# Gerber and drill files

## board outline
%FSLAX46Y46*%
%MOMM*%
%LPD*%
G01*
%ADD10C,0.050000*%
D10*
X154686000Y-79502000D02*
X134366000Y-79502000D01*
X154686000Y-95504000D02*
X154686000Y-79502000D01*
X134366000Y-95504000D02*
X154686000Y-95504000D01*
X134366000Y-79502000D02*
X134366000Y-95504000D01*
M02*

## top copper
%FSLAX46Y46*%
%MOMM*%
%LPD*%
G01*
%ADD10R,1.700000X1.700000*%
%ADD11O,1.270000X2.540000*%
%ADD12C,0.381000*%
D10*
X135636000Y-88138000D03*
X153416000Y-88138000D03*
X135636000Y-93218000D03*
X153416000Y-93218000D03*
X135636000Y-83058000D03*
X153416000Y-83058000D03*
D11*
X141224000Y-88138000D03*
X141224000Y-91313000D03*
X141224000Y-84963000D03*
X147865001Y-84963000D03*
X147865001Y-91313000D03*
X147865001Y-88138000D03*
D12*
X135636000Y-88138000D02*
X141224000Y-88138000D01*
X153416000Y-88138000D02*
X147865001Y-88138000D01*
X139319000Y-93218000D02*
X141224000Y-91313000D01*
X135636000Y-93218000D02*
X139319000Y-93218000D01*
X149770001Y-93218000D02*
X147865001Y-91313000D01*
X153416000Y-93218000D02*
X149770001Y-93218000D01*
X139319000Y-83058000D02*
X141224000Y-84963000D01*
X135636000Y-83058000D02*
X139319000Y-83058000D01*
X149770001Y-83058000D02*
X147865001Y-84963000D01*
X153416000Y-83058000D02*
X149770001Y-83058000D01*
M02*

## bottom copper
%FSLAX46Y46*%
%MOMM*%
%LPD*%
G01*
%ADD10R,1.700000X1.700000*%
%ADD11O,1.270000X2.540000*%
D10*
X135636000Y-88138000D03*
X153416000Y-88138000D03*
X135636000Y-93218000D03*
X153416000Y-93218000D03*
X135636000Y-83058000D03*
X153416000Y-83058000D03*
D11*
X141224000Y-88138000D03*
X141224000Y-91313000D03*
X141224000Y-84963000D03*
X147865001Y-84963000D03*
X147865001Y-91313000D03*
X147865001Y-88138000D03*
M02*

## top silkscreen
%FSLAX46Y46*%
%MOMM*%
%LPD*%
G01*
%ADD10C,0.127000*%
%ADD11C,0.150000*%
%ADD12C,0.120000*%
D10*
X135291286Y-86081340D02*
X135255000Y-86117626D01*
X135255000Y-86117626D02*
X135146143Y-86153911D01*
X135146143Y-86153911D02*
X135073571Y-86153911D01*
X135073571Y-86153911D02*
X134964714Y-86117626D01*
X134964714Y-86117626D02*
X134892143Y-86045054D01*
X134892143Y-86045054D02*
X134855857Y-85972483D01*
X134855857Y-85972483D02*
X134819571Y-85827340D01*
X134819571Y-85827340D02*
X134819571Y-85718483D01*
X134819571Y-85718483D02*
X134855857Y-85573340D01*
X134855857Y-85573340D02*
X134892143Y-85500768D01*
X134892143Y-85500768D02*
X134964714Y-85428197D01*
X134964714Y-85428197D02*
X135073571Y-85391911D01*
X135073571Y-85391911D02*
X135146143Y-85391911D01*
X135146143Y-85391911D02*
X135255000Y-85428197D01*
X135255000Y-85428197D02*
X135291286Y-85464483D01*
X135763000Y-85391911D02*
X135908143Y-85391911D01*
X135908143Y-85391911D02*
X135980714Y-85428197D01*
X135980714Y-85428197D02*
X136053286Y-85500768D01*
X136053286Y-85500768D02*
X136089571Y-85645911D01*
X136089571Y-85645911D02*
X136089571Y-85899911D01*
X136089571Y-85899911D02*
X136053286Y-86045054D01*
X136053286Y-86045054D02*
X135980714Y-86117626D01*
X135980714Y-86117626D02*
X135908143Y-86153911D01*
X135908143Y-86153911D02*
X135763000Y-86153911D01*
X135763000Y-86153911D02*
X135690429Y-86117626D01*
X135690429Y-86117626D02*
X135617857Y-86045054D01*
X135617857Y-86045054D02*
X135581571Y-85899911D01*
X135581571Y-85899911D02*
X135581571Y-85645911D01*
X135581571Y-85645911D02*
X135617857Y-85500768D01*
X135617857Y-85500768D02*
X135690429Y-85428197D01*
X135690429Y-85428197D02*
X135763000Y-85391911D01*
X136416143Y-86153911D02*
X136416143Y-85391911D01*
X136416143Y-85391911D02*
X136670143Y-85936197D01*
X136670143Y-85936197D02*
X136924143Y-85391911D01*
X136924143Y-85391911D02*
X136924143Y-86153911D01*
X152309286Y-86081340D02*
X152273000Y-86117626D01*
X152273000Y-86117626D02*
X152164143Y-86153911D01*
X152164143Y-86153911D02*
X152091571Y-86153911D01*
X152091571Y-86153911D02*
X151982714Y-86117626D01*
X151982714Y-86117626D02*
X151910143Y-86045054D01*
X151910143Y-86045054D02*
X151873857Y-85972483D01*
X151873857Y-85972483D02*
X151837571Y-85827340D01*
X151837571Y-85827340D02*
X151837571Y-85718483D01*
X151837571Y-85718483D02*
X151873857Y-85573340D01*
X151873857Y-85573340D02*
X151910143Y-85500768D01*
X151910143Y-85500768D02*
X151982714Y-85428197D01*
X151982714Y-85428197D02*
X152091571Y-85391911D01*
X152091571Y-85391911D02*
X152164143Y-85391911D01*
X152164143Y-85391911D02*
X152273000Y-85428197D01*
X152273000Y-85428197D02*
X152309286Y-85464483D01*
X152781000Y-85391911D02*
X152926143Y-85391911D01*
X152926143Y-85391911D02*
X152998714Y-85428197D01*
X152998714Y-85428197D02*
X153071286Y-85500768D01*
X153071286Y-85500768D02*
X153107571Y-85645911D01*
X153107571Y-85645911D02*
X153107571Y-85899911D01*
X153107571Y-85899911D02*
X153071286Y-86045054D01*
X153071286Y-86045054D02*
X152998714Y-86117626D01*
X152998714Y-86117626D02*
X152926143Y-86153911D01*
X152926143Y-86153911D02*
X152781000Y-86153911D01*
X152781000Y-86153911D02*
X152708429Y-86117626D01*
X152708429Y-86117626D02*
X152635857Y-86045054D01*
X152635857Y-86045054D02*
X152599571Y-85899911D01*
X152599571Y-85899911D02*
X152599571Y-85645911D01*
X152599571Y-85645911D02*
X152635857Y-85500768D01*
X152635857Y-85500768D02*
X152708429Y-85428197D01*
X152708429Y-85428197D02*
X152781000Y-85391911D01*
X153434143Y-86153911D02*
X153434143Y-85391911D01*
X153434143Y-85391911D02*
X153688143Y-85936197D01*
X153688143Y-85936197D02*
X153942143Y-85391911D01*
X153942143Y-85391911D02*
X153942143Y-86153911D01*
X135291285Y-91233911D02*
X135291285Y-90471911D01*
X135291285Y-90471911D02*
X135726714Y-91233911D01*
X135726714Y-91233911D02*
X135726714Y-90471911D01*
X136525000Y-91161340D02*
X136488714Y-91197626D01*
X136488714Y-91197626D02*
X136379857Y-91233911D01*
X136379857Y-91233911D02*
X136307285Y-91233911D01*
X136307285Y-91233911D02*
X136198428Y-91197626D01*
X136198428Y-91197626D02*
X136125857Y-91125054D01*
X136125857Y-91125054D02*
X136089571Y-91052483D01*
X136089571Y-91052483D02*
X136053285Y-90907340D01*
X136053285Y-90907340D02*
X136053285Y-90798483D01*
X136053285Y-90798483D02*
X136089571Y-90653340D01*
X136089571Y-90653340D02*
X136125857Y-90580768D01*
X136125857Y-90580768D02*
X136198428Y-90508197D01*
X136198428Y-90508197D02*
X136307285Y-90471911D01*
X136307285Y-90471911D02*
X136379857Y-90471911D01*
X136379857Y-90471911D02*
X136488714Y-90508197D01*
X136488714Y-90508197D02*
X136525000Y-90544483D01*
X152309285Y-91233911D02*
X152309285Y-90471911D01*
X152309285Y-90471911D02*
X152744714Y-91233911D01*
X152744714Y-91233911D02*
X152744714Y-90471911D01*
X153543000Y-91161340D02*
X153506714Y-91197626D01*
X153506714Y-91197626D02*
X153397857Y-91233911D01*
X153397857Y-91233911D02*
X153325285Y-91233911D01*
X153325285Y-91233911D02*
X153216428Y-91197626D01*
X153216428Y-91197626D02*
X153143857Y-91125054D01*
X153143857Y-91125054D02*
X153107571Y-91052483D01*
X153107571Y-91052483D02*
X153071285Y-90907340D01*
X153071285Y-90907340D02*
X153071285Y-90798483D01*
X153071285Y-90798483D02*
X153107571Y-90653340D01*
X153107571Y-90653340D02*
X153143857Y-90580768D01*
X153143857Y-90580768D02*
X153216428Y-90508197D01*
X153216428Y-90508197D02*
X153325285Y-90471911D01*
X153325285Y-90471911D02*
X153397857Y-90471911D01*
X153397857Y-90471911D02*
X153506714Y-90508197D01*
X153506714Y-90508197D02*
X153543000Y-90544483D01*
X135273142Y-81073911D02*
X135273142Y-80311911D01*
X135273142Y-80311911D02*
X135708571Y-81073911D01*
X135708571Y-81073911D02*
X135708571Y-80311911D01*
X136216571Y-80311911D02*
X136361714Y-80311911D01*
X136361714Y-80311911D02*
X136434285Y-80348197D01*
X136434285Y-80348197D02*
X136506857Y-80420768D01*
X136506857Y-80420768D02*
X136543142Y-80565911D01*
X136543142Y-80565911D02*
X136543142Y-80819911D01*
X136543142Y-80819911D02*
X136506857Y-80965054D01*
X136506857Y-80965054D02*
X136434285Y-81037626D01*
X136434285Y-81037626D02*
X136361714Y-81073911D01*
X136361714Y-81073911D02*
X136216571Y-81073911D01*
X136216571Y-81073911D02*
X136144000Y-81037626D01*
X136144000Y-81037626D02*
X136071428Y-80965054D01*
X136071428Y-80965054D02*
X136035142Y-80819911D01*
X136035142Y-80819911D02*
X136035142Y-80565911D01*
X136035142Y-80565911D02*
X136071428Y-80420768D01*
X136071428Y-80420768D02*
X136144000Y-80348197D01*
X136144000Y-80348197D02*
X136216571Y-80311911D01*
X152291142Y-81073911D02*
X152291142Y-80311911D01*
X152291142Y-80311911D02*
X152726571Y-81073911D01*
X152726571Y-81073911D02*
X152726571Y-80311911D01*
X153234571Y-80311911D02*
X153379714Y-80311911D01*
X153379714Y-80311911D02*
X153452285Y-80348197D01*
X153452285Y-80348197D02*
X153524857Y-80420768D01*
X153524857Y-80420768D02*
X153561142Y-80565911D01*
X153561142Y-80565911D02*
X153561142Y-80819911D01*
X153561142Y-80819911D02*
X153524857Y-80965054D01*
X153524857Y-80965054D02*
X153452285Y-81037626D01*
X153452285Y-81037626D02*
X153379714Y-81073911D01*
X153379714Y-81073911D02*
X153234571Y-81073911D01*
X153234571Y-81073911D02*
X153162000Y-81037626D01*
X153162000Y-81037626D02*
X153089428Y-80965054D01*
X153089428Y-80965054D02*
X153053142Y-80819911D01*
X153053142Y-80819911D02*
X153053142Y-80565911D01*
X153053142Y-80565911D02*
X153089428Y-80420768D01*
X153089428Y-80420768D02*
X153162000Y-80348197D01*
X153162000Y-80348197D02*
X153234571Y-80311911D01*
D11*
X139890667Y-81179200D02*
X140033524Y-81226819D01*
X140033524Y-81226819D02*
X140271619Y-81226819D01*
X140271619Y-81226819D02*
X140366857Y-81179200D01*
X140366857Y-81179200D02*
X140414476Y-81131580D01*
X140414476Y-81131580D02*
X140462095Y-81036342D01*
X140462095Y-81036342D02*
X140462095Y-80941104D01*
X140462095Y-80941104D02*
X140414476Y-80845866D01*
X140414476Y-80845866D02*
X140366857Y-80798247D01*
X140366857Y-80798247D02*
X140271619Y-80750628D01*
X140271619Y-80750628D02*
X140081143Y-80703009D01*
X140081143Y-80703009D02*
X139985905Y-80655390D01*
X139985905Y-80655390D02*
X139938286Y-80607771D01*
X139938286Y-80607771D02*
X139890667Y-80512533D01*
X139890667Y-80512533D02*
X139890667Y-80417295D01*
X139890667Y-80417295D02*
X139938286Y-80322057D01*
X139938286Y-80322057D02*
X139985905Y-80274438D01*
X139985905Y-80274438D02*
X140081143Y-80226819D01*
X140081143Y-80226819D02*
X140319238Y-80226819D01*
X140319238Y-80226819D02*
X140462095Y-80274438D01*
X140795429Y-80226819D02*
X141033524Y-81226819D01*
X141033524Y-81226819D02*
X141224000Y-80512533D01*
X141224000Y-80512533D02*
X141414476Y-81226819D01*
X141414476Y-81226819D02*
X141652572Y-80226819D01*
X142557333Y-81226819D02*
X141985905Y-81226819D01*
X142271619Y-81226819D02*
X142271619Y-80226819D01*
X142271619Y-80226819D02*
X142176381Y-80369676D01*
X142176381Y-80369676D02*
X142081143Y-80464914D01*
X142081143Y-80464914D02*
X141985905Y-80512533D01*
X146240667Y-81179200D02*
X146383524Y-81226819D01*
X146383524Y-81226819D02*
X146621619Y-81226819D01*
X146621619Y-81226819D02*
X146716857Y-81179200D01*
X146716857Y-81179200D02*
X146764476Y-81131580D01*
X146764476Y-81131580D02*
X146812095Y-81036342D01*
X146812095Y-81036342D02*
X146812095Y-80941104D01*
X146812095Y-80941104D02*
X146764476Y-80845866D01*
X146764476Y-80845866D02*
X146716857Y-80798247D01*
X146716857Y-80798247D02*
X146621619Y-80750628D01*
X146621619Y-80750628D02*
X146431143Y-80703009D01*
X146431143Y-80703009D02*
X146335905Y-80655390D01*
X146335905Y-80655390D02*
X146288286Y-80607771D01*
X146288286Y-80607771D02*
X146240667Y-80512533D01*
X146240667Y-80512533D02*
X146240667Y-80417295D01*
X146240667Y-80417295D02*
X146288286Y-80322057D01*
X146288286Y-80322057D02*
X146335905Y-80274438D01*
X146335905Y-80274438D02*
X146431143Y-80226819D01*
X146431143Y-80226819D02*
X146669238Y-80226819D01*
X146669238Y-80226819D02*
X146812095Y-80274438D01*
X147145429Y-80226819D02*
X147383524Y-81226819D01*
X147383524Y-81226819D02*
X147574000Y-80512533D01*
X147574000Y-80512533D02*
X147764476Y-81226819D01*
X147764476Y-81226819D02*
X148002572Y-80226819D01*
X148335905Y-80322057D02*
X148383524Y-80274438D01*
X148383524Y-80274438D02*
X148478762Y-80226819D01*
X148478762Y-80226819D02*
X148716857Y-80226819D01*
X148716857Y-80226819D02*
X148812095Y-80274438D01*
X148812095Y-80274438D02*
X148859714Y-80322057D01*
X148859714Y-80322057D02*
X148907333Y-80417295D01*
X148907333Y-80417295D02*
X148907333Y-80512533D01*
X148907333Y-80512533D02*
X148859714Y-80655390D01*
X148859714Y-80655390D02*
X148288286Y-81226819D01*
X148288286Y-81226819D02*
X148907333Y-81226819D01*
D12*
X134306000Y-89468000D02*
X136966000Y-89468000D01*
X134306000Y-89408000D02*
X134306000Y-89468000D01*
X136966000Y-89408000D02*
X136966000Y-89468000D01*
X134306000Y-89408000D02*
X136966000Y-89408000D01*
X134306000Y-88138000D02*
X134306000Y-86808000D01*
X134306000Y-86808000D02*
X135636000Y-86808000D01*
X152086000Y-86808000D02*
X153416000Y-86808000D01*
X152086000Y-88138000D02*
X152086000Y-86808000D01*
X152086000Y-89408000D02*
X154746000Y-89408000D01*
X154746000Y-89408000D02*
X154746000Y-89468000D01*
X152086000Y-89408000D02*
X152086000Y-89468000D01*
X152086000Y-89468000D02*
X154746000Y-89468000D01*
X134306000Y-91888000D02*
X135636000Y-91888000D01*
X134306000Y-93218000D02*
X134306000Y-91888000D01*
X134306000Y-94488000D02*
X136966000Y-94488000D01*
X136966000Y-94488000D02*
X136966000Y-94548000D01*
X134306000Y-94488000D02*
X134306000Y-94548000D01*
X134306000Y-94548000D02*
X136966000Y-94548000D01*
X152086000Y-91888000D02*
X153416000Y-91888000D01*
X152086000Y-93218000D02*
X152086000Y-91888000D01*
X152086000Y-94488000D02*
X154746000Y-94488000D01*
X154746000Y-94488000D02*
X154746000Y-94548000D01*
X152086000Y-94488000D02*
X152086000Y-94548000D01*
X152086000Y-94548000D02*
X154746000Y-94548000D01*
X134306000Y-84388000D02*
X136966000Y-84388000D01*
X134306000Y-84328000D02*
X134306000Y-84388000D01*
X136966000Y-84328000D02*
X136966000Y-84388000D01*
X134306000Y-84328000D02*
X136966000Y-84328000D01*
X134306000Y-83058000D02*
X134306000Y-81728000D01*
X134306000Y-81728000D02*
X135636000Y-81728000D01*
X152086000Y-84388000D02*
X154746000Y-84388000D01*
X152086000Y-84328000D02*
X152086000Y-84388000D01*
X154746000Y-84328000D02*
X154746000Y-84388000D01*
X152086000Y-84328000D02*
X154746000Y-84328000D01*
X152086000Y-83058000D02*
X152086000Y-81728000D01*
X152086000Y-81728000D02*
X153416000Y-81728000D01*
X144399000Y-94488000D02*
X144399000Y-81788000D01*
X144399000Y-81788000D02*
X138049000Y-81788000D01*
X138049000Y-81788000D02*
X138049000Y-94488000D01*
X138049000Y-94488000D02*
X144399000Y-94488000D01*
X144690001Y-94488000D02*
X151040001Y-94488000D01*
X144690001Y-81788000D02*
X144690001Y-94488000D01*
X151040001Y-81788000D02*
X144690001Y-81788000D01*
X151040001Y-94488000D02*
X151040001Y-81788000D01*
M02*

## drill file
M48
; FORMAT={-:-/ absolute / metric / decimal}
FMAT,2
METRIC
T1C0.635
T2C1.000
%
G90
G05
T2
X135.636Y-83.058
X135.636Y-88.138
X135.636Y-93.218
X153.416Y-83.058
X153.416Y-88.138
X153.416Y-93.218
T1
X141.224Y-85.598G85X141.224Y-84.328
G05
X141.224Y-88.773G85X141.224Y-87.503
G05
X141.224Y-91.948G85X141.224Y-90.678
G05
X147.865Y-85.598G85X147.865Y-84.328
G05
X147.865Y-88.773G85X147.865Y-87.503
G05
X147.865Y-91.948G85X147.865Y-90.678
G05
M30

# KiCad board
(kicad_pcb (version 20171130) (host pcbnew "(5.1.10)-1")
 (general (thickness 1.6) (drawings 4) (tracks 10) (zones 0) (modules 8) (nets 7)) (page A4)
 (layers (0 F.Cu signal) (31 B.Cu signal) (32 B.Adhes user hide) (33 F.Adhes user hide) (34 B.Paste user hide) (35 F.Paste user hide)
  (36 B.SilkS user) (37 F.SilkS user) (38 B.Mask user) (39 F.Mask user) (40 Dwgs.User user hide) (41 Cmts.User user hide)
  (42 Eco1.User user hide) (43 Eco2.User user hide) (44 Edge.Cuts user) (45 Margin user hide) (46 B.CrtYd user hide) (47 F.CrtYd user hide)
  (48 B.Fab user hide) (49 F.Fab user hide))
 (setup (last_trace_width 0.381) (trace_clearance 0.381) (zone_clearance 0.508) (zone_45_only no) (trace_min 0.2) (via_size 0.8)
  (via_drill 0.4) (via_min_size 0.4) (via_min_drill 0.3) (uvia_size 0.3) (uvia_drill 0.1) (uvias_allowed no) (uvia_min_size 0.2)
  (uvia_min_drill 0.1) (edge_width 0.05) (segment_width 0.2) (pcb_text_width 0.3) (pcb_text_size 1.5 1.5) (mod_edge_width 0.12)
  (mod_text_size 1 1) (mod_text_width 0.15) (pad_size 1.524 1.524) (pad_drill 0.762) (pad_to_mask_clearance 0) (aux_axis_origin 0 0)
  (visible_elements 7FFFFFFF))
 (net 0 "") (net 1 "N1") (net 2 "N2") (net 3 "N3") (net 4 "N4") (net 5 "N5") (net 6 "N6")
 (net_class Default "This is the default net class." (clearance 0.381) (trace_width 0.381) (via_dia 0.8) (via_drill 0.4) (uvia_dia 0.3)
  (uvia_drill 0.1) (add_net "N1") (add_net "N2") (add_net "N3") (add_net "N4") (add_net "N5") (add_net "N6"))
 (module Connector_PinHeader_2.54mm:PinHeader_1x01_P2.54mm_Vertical (layer F.Cu) (at 135.636 88.138)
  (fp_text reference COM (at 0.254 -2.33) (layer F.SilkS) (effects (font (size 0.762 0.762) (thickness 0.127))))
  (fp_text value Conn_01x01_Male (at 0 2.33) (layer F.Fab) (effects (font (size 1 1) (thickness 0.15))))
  (fp_line (start -1.33 1.33) (end 1.33 1.33) (layer F.SilkS) (width 0.12))
  (fp_line (start -1.33 1.27) (end -1.33 1.33) (layer F.SilkS) (width 0.12))
  (fp_line (start 1.33 1.27) (end 1.33 1.33) (layer F.SilkS) (width 0.12))
  (fp_line (start -1.33 1.27) (end 1.33 1.27) (layer F.SilkS) (width 0.12))
  (fp_line (start -1.33 0) (end -1.33 -1.33) (layer F.SilkS) (width 0.12))
  (fp_line (start -1.33 -1.33) (end 0 -1.33) (layer F.SilkS) (width 0.12))
  (pad 1 thru_hole rect (at 0 0) (size 1.7 1.7) (drill 1) (layers *.Cu *.Mask) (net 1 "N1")))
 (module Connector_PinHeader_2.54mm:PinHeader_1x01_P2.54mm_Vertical (layer F.Cu) (at 153.416 88.138)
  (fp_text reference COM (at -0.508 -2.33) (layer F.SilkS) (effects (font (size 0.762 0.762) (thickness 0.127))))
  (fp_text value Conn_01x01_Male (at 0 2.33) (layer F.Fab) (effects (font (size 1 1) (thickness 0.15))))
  (fp_line (start -1.33 -1.33) (end 0 -1.33) (layer F.SilkS) (width 0.12))
  (fp_line (start -1.33 0) (end -1.33 -1.33) (layer F.SilkS) (width 0.12))
  (fp_line (start -1.33 1.27) (end 1.33 1.27) (layer F.SilkS) (width 0.12))
  (fp_line (start 1.33 1.27) (end 1.33 1.33) (layer F.SilkS) (width 0.12))
  (fp_line (start -1.33 1.27) (end -1.33 1.33) (layer F.SilkS) (width 0.12))
  (fp_line (start -1.33 1.33) (end 1.33 1.33) (layer F.SilkS) (width 0.12))
  (pad 1 thru_hole rect (at 0 0) (size 1.7 1.7) (drill 1) (layers *.Cu *.Mask) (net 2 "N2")))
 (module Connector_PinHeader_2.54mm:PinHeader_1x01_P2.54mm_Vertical (layer F.Cu) (at 135.636 93.218)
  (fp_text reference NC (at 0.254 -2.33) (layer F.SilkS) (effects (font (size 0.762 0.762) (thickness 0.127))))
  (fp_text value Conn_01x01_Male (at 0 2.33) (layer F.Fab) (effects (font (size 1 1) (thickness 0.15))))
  (fp_line (start -1.33 -1.33) (end 0 -1.33) (layer F.SilkS) (width 0.12))
  (fp_line (start -1.33 0) (end -1.33 -1.33) (layer F.SilkS) (width 0.12))
  (fp_line (start -1.33 1.27) (end 1.33 1.27) (layer F.SilkS) (width 0.12))
  (fp_line (start 1.33 1.27) (end 1.33 1.33) (layer F.SilkS) (width 0.12))
  (fp_line (start -1.33 1.27) (end -1.33 1.33) (layer F.SilkS) (width 0.12))
  (fp_line (start -1.33 1.33) (end 1.33 1.33) (layer F.SilkS) (width 0.12))
  (pad 1 thru_hole rect (at 0 0) (size 1.7 1.7) (drill 1) (layers *.Cu *.Mask) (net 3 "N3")))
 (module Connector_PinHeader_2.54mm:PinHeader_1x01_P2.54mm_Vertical (layer F.Cu) (at 153.416 93.218)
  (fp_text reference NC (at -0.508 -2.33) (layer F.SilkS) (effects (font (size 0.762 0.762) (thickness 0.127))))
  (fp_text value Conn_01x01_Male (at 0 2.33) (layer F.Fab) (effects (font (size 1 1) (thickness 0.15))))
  (fp_line (start -1.33 -1.33) (end 0 -1.33) (layer F.SilkS) (width 0.12))
  (fp_line (start -1.33 0) (end -1.33 -1.33) (layer F.SilkS) (width 0.12))
  (fp_line (start -1.33 1.27) (end 1.33 1.27) (layer F.SilkS) (width 0.12))
  (fp_line (start 1.33 1.27) (end 1.33 1.33) (layer F.SilkS) (width 0.12))
  (fp_line (start -1.33 1.27) (end -1.33 1.33) (layer F.SilkS) (width 0.12))
  (fp_line (start -1.33 1.33) (end 1.33 1.33) (layer F.SilkS) (width 0.12))
  (pad 1 thru_hole rect (at 0 0) (size 1.7 1.7) (drill 1) (layers *.Cu *.Mask) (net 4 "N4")))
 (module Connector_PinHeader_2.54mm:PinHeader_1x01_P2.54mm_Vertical (layer F.Cu) (at 135.636 83.058)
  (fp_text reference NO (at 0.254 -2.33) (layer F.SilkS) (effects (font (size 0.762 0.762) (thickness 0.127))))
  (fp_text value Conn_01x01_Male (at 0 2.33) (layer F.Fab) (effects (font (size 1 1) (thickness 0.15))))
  (fp_line (start -1.33 1.33) (end 1.33 1.33) (layer F.SilkS) (width 0.12))
  (fp_line (start -1.33 1.27) (end -1.33 1.33) (layer F.SilkS) (width 0.12))
  (fp_line (start 1.33 1.27) (end 1.33 1.33) (layer F.SilkS) (width 0.12))
  (fp_line (start -1.33 1.27) (end 1.33 1.27) (layer F.SilkS) (width 0.12))
  (fp_line (start -1.33 0) (end -1.33 -1.33) (layer F.SilkS) (width 0.12))
  (fp_line (start -1.33 -1.33) (end 0 -1.33) (layer F.SilkS) (width 0.12))
  (pad 1 thru_hole rect (at 0 0) (size 1.7 1.7) (drill 1) (layers *.Cu *.Mask) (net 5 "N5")))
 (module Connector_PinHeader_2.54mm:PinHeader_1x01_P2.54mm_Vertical (layer F.Cu) (at 153.416 83.058)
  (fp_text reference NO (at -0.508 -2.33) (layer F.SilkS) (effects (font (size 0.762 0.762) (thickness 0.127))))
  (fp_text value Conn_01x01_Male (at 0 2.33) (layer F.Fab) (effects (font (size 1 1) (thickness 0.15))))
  (fp_line (start -1.33 1.33) (end 1.33 1.33) (layer F.SilkS) (width 0.12))
  (fp_line (start -1.33 1.27) (end -1.33 1.33) (layer F.SilkS) (width 0.12))
  (fp_line (start 1.33 1.27) (end 1.33 1.33) (layer F.SilkS) (width 0.12))
  (fp_line (start -1.33 1.27) (end 1.33 1.27) (layer F.SilkS) (width 0.12))
  (fp_line (start -1.33 0) (end -1.33 -1.33) (layer F.SilkS) (width 0.12))
  (fp_line (start -1.33 -1.33) (end 0 -1.33) (layer F.SilkS) (width 0.12))
  (pad 1 thru_hole rect (at 0 0) (size 1.7 1.7) (drill 1) (layers *.Cu *.Mask) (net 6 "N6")))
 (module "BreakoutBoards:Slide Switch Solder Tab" (layer F.Cu) (at 141.224 88.138 180)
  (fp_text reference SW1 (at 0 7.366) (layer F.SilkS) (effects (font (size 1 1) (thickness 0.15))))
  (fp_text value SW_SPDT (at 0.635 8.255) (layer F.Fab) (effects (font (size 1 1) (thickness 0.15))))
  (fp_line (start -3.175 -6.35) (end -3.175 6.35) (layer F.SilkS) (width 0.12))
  (fp_line (start -3.175 6.35) (end 3.175 6.35) (layer F.SilkS) (width 0.12))
  (fp_line (start 3.175 6.35) (end 3.175 -6.35) (layer F.SilkS) (width 0.12))
  (fp_line (start 3.175 -6.35) (end -3.175 -6.35) (layer F.SilkS) (width 0.12))
  (pad 2 thru_hole oval (at 0 0 180) (size 1.27 2.54) (drill oval 0.635 1.905) (layers *.Cu *.Mask) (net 1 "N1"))
  (pad 1 thru_hole oval (at 0 -3.175 180) (size 1.27 2.54) (drill oval 0.635 1.905) (layers *.Cu *.Mask) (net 3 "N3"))
  (pad 3 thru_hole oval (at 0 3.175 180) (size 1.27 2.54) (drill oval 0.635 1.905) (layers *.Cu *.Mask) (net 5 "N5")))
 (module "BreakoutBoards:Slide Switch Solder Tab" (layer F.Cu) (at 147.865001 88.138 180)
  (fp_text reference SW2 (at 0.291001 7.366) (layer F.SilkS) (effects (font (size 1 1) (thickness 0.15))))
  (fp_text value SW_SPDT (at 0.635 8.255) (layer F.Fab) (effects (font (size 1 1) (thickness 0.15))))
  (fp_line (start 3.175 -6.35) (end -3.175 -6.35) (layer F.SilkS) (width 0.12))
  (fp_line (start 3.175 6.35) (end 3.175 -6.35) (layer F.SilkS) (width 0.12))
  (fp_line (start -3.175 6.35) (end 3.175 6.35) (layer F.SilkS) (width 0.12))
  (fp_line (start -3.175 -6.35) (end -3.175 6.35) (layer F.SilkS) (width 0.12))
  (pad 3 thru_hole oval (at 0 3.175 180) (size 1.27 2.54) (drill oval 0.635 1.905) (layers *.Cu *.Mask) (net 6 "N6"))
  (pad 1 thru_hole oval (at 0 -3.175 180) (size 1.27 2.54) (drill oval 0.635 1.905) (layers *.Cu *.Mask) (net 4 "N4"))
  (pad 2 thru_hole oval (at 0 0 180) (size 1.27 2.54) (drill oval 0.635 1.905) (layers *.Cu *.Mask) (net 2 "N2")))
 (gr_line (start 154.686 79.502) (end 134.366 79.502) (layer Edge.Cuts) (width 0.05))
 (gr_line (start 154.686 95.504) (end 154.686 79.502) (layer Edge.Cuts) (width 0.05))
 (gr_line (start 134.366 95.504) (end 154.686 95.504) (layer Edge.Cuts) (width 0.05))
 (gr_line (start 134.366 79.502) (end 134.366 95.504) (layer Edge.Cuts) (width 0.05))
 (segment (start 135.636 88.138) (end 141.224 88.138) (width 0.381) (layer F.Cu) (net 1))
 (segment (start 153.416 88.138) (end 147.865001 88.138) (width 0.381) (layer F.Cu) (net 2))
 (segment (start 139.319 93.218) (end 141.224 91.313) (width 0.381) (layer F.Cu) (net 3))
 (segment (start 135.636 93.218) (end 139.319 93.218) (width 0.381) (layer F.Cu) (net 3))
 (segment (start 149.770001 93.218) (end 147.865001 91.313) (width 0.381) (layer F.Cu) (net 4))
 (segment (start 153.416 93.218) (end 149.770001 93.218) (width 0.381) (layer F.Cu) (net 4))
 (segment (start 139.319 83.058) (end 141.224 84.963) (width 0.381) (layer F.Cu) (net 5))
 (segment (start 135.636 83.058) (end 139.319 83.058) (width 0.381) (layer F.Cu) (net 5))
 (segment (start 149.770001 83.058) (end 147.865001 84.963) (width 0.381) (layer F.Cu) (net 6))
 (segment (start 153.416 83.058) (end 149.770001 83.058) (width 0.381) (layer F.Cu) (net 6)))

